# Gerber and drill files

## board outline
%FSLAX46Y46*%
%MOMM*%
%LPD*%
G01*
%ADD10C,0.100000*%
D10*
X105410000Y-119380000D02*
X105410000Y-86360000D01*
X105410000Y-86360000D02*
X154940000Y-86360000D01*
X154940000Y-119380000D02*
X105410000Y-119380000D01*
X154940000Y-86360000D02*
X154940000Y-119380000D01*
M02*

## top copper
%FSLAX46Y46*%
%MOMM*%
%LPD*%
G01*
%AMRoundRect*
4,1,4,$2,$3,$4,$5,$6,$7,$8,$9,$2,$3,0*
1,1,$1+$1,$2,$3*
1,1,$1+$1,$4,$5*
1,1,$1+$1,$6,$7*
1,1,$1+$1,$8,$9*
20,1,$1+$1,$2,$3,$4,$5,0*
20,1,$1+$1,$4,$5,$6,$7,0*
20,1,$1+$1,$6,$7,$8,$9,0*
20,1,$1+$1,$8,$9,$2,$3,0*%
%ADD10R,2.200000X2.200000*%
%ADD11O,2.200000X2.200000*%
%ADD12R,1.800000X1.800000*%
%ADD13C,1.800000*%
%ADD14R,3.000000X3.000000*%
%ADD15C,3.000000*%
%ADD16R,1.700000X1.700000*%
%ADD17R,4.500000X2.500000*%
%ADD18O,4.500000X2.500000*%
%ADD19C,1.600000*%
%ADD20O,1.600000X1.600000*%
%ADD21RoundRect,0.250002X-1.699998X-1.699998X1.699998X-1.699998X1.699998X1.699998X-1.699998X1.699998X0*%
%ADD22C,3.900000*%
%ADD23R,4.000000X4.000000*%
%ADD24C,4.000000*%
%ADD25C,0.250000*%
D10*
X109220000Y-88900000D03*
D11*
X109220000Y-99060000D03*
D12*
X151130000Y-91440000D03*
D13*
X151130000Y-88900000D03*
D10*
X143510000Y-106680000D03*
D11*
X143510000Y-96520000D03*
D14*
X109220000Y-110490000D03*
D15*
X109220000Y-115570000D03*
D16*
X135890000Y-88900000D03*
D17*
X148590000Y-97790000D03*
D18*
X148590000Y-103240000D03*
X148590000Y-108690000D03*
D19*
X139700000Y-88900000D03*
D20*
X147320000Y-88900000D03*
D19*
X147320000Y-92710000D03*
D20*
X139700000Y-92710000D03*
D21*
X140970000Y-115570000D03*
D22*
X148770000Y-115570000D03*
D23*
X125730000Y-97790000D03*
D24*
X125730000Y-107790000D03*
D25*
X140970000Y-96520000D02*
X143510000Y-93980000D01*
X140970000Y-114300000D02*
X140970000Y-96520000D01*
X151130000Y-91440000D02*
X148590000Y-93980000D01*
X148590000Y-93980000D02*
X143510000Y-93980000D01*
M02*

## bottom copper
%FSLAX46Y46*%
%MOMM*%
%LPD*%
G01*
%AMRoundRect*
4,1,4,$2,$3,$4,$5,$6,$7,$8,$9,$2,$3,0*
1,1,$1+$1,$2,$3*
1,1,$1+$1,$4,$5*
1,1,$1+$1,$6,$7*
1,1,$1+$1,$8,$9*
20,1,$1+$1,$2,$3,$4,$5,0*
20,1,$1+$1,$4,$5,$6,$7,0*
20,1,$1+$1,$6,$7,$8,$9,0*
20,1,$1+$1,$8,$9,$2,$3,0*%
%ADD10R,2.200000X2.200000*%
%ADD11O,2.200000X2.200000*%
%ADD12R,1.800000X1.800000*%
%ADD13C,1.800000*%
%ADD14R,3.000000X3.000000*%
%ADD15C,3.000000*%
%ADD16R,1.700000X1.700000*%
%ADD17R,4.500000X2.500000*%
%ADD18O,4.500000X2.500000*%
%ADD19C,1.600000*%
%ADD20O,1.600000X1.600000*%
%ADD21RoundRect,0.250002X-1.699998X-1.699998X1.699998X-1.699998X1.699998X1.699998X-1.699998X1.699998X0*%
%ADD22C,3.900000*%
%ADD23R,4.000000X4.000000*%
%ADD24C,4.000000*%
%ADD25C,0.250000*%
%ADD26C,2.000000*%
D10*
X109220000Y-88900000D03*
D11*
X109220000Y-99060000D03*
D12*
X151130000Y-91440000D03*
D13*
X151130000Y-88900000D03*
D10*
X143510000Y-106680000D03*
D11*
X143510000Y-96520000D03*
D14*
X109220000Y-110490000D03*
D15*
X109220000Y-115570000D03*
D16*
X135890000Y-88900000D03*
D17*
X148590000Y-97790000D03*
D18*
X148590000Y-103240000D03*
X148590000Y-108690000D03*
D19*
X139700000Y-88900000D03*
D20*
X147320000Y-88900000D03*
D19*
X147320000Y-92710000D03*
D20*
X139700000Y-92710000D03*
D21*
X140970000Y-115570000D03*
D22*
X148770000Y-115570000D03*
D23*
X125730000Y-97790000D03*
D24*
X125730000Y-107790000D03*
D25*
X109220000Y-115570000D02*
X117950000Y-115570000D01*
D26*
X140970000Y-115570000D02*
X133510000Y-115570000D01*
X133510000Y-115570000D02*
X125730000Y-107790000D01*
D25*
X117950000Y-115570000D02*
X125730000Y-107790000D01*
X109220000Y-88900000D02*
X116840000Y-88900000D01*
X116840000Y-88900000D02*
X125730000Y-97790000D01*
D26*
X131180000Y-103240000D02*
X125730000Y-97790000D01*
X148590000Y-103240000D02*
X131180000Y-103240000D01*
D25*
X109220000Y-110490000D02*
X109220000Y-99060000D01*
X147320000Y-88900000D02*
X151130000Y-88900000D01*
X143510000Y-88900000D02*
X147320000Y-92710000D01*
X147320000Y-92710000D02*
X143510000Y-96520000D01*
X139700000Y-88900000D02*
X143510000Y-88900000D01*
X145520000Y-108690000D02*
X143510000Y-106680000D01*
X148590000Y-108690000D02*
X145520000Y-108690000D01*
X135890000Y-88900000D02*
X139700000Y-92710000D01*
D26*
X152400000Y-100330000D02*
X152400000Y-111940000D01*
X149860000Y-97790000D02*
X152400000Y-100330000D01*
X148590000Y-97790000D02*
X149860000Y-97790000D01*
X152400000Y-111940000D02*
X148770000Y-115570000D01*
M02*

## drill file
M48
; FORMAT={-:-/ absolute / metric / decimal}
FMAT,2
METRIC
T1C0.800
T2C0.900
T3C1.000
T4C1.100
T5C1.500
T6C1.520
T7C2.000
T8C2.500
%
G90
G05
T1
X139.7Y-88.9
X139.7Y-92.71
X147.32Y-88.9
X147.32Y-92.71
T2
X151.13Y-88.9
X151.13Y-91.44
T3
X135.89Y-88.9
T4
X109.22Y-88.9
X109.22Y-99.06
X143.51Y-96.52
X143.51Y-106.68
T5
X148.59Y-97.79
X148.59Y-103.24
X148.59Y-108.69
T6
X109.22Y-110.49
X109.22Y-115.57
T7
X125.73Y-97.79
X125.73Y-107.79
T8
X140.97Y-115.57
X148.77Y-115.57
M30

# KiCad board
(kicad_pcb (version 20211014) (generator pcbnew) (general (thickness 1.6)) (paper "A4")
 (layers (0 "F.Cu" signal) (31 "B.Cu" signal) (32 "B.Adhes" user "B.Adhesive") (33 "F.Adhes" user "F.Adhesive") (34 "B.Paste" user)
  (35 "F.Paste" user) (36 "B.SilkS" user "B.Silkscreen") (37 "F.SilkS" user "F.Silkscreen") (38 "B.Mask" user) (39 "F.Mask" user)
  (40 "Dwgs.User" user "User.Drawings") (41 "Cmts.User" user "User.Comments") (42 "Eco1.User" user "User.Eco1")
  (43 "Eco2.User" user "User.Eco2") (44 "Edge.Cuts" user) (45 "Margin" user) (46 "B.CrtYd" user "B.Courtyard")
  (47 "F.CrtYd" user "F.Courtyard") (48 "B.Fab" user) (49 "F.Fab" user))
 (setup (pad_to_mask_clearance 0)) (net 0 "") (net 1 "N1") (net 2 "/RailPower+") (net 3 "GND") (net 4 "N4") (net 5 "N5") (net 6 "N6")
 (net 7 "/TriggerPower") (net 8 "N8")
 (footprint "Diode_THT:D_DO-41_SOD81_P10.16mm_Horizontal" (layer "F.Cu") (at 109.22 88.9 -90)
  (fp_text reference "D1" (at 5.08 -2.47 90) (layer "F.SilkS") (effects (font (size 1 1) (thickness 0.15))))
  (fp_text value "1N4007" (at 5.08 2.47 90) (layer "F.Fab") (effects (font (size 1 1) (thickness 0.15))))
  (pad "1" thru_hole rect (at 0 0 270) (size 2.2 2.2) (drill 1.1) (layers *.Cu *.Mask) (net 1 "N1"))
  (pad "2" thru_hole oval (at 10.16 0 270) (size 2.2 2.2) (drill 1.1) (layers *.Cu *.Mask) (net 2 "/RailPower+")))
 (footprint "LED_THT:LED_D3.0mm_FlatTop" (layer "F.Cu") (at 151.13 91.44 90)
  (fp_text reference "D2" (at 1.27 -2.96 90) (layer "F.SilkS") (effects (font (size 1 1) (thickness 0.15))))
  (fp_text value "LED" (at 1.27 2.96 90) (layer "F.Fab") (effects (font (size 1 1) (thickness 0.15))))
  (pad "1" thru_hole rect (at 0 0 90) (size 1.8 1.8) (drill 0.9) (layers *.Cu *.Mask) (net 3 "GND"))
  (pad "2" thru_hole circle (at 2.54 0 90) (size 1.8 1.8) (drill 0.9) (layers *.Cu *.Mask) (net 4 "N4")))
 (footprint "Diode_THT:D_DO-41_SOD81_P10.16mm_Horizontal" (layer "F.Cu") (at 143.51 106.68 90)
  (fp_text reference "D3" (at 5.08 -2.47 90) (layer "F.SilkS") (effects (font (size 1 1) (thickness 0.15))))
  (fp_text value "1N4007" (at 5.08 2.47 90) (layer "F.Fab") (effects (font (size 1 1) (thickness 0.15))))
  (pad "1" thru_hole rect (at 0 0 90) (size 2.2 2.2) (drill 1.1) (layers *.Cu *.Mask) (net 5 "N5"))
  (pad "2" thru_hole oval (at 10.16 0 90) (size 2.2 2.2) (drill 1.1) (layers *.Cu *.Mask) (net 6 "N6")))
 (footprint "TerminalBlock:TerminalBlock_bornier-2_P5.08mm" (layer "F.Cu") (at 109.22 110.49 -90)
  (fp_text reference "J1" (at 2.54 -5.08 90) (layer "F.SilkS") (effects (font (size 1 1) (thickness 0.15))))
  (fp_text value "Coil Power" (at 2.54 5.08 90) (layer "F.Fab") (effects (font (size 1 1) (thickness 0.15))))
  (pad "1" thru_hole rect (at 0 0 270) (size 3 3) (drill 1.52) (layers *.Cu *.Mask) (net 2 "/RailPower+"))
  (pad "2" thru_hole circle (at 5.08 0 270) (size 3 3) (drill 1.52) (layers *.Cu *.Mask) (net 3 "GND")))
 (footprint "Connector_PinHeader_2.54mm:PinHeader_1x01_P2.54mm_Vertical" (layer "F.Cu") (at 135.89 88.9)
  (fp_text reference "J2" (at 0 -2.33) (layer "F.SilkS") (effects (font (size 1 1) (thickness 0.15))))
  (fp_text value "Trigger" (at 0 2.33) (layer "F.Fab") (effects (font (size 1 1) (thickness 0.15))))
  (pad "1" thru_hole rect (at 0 0) (size 1.7 1.7) (drill 1) (layers *.Cu *.Mask) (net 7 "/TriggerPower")))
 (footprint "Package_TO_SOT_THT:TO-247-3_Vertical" (layer "F.Cu") (at 148.59 97.79 -90)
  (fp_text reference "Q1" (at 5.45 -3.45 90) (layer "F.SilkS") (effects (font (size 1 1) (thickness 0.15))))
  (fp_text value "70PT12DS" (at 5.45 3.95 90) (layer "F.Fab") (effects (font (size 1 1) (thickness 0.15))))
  (pad "1" thru_hole rect (at 0 0 270) (size 2.5 4.5) (drill 1.5) (layers *.Cu *.Mask) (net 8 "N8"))
  (pad "2" thru_hole oval (at 5.45 0 270) (size 2.5 4.5) (drill 1.5) (layers *.Cu *.Mask) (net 1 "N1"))
  (pad "3" thru_hole oval (at 10.9 0 270) (size 2.5 4.5) (drill 1.5) (layers *.Cu *.Mask) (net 5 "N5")))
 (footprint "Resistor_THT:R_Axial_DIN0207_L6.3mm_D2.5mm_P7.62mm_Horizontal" (layer "F.Cu") (at 139.7 88.9)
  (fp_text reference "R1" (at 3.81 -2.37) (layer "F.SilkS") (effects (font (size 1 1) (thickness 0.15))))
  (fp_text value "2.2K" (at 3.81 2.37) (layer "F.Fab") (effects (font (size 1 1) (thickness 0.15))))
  (pad "1" thru_hole circle (at 0 0) (size 1.6 1.6) (drill 0.8) (layers *.Cu *.Mask) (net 6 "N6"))
  (pad "2" thru_hole oval (at 7.62 0) (size 1.6 1.6) (drill 0.8) (layers *.Cu *.Mask) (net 4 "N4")))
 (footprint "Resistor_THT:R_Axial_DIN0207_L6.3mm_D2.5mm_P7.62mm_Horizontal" (layer "F.Cu") (at 147.32 92.71 180)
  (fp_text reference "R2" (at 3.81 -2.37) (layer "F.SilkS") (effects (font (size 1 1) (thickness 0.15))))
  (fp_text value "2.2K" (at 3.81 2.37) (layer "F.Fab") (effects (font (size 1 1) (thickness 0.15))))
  (pad "1" thru_hole circle (at 0 0 180) (size 1.6 1.6) (drill 0.8) (layers *.Cu *.Mask) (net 6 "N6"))
  (pad "2" thru_hole oval (at 7.62 0 180) (size 1.6 1.6) (drill 0.8) (layers *.Cu *.Mask) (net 7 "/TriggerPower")))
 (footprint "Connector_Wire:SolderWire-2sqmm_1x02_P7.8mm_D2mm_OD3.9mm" (layer "F.Cu") (at 140.97 115.57)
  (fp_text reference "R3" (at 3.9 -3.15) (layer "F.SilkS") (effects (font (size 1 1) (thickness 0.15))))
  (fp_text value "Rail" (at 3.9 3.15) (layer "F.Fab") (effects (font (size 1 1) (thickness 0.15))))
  (pad "1" thru_hole roundrect (at 0 0) (size 3.9 3.9) (drill 2.5) (layers *.Cu *.Mask) (roundrect_rratio 0.064103) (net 3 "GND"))
  (pad "2" thru_hole circle (at 7.8 0) (size 3.9 3.9) (drill 2.5) (layers *.Cu *.Mask) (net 8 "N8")))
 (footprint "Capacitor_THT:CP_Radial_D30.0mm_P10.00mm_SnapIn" (layer "B.Cu") (at 125.73 97.79 -90)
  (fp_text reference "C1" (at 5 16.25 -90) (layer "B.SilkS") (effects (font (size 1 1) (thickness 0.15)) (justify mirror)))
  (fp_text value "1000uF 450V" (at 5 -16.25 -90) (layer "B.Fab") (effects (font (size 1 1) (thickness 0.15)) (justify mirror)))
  (pad "1" thru_hole rect (at 0 0 270) (size 4 4) (drill 2) (layers *.Cu *.Mask) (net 1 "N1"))
  (pad "2" thru_hole circle (at 10 0 270) (size 4 4) (drill 2) (layers *.Cu *.Mask) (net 3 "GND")))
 (gr_line (start 105.41 119.38) (end 105.41 86.36) (layer "Edge.Cuts") (width 0.1))
 (gr_line (start 105.41 86.36) (end 154.94 86.36) (layer "Edge.Cuts") (width 0.1))
 (gr_line (start 154.94 119.38) (end 105.41 119.38) (layer "Edge.Cuts") (width 0.1))
 (gr_line (start 154.94 86.36) (end 154.94 119.38) (layer "Edge.Cuts") (width 0.1))
 (segment (start 140.97 96.52) (end 143.51 93.98) (width 0.25) (layer "F.Cu") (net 3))
 (segment (start 140.97 114.3) (end 140.97 96.52) (width 0.25) (layer "F.Cu") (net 3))
 (segment (start 151.13 91.44) (end 148.59 93.98) (width 0.25) (layer "F.Cu") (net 3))
 (segment (start 148.59 93.98) (end 143.51 93.98) (width 0.25) (layer "F.Cu") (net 3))
 (segment (start 109.22 115.57) (end 117.95 115.57) (width 0.25) (layer "B.Cu") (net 3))
 (segment (start 140.97 115.57) (end 133.51 115.57) (width 2) (layer "B.Cu") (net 3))
 (segment (start 133.51 115.57) (end 125.73 107.79) (width 2) (layer "B.Cu") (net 3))
 (segment (start 117.95 115.57) (end 125.73 107.79) (width 0.25) (layer "B.Cu") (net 3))
 (segment (start 109.22 88.9) (end 116.84 88.9) (width 0.25) (layer "B.Cu") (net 1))
 (segment (start 116.84 88.9) (end 125.73 97.79) (width 0.25) (layer "B.Cu") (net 1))
 (segment (start 131.18 103.24) (end 125.73 97.79) (width 2) (layer "B.Cu") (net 1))
 (segment (start 148.59 103.24) (end 131.18 103.24) (width 2) (layer "B.Cu") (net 1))
 (segment (start 109.22 110.49) (end 109.22 99.06) (width 0.25) (layer "B.Cu") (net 2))
 (segment (start 147.32 88.9) (end 151.13 88.9) (width 0.25) (layer "B.Cu") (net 4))
 (segment (start 143.51 88.9) (end 147.32 92.71) (width 0.25) (layer "B.Cu") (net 6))
 (segment (start 147.32 92.71) (end 143.51 96.52) (width 0.25) (layer "B.Cu") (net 6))
 (segment (start 139.7 88.9) (end 143.51 88.9) (width 0.25) (layer "B.Cu") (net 6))
 (segment (start 145.52 108.69) (end 143.51 106.68) (width 0.25) (layer "B.Cu") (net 5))
 (segment (start 148.59 108.69) (end 145.52 108.69) (width 0.25) (layer "B.Cu") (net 5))
 (segment (start 135.89 88.9) (end 139.7 92.71) (width 0.25) (layer "B.Cu") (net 7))
 (segment (start 152.4 100.33) (end 152.4 111.94) (width 2) (layer "B.Cu") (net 8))
 (segment (start 149.86 97.79) (end 152.4 100.33) (width 2) (layer "B.Cu") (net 8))
 (segment (start 148.59 97.79) (end 149.86 97.79) (width 2) (layer "B.Cu") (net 8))
 (segment (start 152.4 111.94) (end 148.77 115.57) (width 2) (layer "B.Cu") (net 8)))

